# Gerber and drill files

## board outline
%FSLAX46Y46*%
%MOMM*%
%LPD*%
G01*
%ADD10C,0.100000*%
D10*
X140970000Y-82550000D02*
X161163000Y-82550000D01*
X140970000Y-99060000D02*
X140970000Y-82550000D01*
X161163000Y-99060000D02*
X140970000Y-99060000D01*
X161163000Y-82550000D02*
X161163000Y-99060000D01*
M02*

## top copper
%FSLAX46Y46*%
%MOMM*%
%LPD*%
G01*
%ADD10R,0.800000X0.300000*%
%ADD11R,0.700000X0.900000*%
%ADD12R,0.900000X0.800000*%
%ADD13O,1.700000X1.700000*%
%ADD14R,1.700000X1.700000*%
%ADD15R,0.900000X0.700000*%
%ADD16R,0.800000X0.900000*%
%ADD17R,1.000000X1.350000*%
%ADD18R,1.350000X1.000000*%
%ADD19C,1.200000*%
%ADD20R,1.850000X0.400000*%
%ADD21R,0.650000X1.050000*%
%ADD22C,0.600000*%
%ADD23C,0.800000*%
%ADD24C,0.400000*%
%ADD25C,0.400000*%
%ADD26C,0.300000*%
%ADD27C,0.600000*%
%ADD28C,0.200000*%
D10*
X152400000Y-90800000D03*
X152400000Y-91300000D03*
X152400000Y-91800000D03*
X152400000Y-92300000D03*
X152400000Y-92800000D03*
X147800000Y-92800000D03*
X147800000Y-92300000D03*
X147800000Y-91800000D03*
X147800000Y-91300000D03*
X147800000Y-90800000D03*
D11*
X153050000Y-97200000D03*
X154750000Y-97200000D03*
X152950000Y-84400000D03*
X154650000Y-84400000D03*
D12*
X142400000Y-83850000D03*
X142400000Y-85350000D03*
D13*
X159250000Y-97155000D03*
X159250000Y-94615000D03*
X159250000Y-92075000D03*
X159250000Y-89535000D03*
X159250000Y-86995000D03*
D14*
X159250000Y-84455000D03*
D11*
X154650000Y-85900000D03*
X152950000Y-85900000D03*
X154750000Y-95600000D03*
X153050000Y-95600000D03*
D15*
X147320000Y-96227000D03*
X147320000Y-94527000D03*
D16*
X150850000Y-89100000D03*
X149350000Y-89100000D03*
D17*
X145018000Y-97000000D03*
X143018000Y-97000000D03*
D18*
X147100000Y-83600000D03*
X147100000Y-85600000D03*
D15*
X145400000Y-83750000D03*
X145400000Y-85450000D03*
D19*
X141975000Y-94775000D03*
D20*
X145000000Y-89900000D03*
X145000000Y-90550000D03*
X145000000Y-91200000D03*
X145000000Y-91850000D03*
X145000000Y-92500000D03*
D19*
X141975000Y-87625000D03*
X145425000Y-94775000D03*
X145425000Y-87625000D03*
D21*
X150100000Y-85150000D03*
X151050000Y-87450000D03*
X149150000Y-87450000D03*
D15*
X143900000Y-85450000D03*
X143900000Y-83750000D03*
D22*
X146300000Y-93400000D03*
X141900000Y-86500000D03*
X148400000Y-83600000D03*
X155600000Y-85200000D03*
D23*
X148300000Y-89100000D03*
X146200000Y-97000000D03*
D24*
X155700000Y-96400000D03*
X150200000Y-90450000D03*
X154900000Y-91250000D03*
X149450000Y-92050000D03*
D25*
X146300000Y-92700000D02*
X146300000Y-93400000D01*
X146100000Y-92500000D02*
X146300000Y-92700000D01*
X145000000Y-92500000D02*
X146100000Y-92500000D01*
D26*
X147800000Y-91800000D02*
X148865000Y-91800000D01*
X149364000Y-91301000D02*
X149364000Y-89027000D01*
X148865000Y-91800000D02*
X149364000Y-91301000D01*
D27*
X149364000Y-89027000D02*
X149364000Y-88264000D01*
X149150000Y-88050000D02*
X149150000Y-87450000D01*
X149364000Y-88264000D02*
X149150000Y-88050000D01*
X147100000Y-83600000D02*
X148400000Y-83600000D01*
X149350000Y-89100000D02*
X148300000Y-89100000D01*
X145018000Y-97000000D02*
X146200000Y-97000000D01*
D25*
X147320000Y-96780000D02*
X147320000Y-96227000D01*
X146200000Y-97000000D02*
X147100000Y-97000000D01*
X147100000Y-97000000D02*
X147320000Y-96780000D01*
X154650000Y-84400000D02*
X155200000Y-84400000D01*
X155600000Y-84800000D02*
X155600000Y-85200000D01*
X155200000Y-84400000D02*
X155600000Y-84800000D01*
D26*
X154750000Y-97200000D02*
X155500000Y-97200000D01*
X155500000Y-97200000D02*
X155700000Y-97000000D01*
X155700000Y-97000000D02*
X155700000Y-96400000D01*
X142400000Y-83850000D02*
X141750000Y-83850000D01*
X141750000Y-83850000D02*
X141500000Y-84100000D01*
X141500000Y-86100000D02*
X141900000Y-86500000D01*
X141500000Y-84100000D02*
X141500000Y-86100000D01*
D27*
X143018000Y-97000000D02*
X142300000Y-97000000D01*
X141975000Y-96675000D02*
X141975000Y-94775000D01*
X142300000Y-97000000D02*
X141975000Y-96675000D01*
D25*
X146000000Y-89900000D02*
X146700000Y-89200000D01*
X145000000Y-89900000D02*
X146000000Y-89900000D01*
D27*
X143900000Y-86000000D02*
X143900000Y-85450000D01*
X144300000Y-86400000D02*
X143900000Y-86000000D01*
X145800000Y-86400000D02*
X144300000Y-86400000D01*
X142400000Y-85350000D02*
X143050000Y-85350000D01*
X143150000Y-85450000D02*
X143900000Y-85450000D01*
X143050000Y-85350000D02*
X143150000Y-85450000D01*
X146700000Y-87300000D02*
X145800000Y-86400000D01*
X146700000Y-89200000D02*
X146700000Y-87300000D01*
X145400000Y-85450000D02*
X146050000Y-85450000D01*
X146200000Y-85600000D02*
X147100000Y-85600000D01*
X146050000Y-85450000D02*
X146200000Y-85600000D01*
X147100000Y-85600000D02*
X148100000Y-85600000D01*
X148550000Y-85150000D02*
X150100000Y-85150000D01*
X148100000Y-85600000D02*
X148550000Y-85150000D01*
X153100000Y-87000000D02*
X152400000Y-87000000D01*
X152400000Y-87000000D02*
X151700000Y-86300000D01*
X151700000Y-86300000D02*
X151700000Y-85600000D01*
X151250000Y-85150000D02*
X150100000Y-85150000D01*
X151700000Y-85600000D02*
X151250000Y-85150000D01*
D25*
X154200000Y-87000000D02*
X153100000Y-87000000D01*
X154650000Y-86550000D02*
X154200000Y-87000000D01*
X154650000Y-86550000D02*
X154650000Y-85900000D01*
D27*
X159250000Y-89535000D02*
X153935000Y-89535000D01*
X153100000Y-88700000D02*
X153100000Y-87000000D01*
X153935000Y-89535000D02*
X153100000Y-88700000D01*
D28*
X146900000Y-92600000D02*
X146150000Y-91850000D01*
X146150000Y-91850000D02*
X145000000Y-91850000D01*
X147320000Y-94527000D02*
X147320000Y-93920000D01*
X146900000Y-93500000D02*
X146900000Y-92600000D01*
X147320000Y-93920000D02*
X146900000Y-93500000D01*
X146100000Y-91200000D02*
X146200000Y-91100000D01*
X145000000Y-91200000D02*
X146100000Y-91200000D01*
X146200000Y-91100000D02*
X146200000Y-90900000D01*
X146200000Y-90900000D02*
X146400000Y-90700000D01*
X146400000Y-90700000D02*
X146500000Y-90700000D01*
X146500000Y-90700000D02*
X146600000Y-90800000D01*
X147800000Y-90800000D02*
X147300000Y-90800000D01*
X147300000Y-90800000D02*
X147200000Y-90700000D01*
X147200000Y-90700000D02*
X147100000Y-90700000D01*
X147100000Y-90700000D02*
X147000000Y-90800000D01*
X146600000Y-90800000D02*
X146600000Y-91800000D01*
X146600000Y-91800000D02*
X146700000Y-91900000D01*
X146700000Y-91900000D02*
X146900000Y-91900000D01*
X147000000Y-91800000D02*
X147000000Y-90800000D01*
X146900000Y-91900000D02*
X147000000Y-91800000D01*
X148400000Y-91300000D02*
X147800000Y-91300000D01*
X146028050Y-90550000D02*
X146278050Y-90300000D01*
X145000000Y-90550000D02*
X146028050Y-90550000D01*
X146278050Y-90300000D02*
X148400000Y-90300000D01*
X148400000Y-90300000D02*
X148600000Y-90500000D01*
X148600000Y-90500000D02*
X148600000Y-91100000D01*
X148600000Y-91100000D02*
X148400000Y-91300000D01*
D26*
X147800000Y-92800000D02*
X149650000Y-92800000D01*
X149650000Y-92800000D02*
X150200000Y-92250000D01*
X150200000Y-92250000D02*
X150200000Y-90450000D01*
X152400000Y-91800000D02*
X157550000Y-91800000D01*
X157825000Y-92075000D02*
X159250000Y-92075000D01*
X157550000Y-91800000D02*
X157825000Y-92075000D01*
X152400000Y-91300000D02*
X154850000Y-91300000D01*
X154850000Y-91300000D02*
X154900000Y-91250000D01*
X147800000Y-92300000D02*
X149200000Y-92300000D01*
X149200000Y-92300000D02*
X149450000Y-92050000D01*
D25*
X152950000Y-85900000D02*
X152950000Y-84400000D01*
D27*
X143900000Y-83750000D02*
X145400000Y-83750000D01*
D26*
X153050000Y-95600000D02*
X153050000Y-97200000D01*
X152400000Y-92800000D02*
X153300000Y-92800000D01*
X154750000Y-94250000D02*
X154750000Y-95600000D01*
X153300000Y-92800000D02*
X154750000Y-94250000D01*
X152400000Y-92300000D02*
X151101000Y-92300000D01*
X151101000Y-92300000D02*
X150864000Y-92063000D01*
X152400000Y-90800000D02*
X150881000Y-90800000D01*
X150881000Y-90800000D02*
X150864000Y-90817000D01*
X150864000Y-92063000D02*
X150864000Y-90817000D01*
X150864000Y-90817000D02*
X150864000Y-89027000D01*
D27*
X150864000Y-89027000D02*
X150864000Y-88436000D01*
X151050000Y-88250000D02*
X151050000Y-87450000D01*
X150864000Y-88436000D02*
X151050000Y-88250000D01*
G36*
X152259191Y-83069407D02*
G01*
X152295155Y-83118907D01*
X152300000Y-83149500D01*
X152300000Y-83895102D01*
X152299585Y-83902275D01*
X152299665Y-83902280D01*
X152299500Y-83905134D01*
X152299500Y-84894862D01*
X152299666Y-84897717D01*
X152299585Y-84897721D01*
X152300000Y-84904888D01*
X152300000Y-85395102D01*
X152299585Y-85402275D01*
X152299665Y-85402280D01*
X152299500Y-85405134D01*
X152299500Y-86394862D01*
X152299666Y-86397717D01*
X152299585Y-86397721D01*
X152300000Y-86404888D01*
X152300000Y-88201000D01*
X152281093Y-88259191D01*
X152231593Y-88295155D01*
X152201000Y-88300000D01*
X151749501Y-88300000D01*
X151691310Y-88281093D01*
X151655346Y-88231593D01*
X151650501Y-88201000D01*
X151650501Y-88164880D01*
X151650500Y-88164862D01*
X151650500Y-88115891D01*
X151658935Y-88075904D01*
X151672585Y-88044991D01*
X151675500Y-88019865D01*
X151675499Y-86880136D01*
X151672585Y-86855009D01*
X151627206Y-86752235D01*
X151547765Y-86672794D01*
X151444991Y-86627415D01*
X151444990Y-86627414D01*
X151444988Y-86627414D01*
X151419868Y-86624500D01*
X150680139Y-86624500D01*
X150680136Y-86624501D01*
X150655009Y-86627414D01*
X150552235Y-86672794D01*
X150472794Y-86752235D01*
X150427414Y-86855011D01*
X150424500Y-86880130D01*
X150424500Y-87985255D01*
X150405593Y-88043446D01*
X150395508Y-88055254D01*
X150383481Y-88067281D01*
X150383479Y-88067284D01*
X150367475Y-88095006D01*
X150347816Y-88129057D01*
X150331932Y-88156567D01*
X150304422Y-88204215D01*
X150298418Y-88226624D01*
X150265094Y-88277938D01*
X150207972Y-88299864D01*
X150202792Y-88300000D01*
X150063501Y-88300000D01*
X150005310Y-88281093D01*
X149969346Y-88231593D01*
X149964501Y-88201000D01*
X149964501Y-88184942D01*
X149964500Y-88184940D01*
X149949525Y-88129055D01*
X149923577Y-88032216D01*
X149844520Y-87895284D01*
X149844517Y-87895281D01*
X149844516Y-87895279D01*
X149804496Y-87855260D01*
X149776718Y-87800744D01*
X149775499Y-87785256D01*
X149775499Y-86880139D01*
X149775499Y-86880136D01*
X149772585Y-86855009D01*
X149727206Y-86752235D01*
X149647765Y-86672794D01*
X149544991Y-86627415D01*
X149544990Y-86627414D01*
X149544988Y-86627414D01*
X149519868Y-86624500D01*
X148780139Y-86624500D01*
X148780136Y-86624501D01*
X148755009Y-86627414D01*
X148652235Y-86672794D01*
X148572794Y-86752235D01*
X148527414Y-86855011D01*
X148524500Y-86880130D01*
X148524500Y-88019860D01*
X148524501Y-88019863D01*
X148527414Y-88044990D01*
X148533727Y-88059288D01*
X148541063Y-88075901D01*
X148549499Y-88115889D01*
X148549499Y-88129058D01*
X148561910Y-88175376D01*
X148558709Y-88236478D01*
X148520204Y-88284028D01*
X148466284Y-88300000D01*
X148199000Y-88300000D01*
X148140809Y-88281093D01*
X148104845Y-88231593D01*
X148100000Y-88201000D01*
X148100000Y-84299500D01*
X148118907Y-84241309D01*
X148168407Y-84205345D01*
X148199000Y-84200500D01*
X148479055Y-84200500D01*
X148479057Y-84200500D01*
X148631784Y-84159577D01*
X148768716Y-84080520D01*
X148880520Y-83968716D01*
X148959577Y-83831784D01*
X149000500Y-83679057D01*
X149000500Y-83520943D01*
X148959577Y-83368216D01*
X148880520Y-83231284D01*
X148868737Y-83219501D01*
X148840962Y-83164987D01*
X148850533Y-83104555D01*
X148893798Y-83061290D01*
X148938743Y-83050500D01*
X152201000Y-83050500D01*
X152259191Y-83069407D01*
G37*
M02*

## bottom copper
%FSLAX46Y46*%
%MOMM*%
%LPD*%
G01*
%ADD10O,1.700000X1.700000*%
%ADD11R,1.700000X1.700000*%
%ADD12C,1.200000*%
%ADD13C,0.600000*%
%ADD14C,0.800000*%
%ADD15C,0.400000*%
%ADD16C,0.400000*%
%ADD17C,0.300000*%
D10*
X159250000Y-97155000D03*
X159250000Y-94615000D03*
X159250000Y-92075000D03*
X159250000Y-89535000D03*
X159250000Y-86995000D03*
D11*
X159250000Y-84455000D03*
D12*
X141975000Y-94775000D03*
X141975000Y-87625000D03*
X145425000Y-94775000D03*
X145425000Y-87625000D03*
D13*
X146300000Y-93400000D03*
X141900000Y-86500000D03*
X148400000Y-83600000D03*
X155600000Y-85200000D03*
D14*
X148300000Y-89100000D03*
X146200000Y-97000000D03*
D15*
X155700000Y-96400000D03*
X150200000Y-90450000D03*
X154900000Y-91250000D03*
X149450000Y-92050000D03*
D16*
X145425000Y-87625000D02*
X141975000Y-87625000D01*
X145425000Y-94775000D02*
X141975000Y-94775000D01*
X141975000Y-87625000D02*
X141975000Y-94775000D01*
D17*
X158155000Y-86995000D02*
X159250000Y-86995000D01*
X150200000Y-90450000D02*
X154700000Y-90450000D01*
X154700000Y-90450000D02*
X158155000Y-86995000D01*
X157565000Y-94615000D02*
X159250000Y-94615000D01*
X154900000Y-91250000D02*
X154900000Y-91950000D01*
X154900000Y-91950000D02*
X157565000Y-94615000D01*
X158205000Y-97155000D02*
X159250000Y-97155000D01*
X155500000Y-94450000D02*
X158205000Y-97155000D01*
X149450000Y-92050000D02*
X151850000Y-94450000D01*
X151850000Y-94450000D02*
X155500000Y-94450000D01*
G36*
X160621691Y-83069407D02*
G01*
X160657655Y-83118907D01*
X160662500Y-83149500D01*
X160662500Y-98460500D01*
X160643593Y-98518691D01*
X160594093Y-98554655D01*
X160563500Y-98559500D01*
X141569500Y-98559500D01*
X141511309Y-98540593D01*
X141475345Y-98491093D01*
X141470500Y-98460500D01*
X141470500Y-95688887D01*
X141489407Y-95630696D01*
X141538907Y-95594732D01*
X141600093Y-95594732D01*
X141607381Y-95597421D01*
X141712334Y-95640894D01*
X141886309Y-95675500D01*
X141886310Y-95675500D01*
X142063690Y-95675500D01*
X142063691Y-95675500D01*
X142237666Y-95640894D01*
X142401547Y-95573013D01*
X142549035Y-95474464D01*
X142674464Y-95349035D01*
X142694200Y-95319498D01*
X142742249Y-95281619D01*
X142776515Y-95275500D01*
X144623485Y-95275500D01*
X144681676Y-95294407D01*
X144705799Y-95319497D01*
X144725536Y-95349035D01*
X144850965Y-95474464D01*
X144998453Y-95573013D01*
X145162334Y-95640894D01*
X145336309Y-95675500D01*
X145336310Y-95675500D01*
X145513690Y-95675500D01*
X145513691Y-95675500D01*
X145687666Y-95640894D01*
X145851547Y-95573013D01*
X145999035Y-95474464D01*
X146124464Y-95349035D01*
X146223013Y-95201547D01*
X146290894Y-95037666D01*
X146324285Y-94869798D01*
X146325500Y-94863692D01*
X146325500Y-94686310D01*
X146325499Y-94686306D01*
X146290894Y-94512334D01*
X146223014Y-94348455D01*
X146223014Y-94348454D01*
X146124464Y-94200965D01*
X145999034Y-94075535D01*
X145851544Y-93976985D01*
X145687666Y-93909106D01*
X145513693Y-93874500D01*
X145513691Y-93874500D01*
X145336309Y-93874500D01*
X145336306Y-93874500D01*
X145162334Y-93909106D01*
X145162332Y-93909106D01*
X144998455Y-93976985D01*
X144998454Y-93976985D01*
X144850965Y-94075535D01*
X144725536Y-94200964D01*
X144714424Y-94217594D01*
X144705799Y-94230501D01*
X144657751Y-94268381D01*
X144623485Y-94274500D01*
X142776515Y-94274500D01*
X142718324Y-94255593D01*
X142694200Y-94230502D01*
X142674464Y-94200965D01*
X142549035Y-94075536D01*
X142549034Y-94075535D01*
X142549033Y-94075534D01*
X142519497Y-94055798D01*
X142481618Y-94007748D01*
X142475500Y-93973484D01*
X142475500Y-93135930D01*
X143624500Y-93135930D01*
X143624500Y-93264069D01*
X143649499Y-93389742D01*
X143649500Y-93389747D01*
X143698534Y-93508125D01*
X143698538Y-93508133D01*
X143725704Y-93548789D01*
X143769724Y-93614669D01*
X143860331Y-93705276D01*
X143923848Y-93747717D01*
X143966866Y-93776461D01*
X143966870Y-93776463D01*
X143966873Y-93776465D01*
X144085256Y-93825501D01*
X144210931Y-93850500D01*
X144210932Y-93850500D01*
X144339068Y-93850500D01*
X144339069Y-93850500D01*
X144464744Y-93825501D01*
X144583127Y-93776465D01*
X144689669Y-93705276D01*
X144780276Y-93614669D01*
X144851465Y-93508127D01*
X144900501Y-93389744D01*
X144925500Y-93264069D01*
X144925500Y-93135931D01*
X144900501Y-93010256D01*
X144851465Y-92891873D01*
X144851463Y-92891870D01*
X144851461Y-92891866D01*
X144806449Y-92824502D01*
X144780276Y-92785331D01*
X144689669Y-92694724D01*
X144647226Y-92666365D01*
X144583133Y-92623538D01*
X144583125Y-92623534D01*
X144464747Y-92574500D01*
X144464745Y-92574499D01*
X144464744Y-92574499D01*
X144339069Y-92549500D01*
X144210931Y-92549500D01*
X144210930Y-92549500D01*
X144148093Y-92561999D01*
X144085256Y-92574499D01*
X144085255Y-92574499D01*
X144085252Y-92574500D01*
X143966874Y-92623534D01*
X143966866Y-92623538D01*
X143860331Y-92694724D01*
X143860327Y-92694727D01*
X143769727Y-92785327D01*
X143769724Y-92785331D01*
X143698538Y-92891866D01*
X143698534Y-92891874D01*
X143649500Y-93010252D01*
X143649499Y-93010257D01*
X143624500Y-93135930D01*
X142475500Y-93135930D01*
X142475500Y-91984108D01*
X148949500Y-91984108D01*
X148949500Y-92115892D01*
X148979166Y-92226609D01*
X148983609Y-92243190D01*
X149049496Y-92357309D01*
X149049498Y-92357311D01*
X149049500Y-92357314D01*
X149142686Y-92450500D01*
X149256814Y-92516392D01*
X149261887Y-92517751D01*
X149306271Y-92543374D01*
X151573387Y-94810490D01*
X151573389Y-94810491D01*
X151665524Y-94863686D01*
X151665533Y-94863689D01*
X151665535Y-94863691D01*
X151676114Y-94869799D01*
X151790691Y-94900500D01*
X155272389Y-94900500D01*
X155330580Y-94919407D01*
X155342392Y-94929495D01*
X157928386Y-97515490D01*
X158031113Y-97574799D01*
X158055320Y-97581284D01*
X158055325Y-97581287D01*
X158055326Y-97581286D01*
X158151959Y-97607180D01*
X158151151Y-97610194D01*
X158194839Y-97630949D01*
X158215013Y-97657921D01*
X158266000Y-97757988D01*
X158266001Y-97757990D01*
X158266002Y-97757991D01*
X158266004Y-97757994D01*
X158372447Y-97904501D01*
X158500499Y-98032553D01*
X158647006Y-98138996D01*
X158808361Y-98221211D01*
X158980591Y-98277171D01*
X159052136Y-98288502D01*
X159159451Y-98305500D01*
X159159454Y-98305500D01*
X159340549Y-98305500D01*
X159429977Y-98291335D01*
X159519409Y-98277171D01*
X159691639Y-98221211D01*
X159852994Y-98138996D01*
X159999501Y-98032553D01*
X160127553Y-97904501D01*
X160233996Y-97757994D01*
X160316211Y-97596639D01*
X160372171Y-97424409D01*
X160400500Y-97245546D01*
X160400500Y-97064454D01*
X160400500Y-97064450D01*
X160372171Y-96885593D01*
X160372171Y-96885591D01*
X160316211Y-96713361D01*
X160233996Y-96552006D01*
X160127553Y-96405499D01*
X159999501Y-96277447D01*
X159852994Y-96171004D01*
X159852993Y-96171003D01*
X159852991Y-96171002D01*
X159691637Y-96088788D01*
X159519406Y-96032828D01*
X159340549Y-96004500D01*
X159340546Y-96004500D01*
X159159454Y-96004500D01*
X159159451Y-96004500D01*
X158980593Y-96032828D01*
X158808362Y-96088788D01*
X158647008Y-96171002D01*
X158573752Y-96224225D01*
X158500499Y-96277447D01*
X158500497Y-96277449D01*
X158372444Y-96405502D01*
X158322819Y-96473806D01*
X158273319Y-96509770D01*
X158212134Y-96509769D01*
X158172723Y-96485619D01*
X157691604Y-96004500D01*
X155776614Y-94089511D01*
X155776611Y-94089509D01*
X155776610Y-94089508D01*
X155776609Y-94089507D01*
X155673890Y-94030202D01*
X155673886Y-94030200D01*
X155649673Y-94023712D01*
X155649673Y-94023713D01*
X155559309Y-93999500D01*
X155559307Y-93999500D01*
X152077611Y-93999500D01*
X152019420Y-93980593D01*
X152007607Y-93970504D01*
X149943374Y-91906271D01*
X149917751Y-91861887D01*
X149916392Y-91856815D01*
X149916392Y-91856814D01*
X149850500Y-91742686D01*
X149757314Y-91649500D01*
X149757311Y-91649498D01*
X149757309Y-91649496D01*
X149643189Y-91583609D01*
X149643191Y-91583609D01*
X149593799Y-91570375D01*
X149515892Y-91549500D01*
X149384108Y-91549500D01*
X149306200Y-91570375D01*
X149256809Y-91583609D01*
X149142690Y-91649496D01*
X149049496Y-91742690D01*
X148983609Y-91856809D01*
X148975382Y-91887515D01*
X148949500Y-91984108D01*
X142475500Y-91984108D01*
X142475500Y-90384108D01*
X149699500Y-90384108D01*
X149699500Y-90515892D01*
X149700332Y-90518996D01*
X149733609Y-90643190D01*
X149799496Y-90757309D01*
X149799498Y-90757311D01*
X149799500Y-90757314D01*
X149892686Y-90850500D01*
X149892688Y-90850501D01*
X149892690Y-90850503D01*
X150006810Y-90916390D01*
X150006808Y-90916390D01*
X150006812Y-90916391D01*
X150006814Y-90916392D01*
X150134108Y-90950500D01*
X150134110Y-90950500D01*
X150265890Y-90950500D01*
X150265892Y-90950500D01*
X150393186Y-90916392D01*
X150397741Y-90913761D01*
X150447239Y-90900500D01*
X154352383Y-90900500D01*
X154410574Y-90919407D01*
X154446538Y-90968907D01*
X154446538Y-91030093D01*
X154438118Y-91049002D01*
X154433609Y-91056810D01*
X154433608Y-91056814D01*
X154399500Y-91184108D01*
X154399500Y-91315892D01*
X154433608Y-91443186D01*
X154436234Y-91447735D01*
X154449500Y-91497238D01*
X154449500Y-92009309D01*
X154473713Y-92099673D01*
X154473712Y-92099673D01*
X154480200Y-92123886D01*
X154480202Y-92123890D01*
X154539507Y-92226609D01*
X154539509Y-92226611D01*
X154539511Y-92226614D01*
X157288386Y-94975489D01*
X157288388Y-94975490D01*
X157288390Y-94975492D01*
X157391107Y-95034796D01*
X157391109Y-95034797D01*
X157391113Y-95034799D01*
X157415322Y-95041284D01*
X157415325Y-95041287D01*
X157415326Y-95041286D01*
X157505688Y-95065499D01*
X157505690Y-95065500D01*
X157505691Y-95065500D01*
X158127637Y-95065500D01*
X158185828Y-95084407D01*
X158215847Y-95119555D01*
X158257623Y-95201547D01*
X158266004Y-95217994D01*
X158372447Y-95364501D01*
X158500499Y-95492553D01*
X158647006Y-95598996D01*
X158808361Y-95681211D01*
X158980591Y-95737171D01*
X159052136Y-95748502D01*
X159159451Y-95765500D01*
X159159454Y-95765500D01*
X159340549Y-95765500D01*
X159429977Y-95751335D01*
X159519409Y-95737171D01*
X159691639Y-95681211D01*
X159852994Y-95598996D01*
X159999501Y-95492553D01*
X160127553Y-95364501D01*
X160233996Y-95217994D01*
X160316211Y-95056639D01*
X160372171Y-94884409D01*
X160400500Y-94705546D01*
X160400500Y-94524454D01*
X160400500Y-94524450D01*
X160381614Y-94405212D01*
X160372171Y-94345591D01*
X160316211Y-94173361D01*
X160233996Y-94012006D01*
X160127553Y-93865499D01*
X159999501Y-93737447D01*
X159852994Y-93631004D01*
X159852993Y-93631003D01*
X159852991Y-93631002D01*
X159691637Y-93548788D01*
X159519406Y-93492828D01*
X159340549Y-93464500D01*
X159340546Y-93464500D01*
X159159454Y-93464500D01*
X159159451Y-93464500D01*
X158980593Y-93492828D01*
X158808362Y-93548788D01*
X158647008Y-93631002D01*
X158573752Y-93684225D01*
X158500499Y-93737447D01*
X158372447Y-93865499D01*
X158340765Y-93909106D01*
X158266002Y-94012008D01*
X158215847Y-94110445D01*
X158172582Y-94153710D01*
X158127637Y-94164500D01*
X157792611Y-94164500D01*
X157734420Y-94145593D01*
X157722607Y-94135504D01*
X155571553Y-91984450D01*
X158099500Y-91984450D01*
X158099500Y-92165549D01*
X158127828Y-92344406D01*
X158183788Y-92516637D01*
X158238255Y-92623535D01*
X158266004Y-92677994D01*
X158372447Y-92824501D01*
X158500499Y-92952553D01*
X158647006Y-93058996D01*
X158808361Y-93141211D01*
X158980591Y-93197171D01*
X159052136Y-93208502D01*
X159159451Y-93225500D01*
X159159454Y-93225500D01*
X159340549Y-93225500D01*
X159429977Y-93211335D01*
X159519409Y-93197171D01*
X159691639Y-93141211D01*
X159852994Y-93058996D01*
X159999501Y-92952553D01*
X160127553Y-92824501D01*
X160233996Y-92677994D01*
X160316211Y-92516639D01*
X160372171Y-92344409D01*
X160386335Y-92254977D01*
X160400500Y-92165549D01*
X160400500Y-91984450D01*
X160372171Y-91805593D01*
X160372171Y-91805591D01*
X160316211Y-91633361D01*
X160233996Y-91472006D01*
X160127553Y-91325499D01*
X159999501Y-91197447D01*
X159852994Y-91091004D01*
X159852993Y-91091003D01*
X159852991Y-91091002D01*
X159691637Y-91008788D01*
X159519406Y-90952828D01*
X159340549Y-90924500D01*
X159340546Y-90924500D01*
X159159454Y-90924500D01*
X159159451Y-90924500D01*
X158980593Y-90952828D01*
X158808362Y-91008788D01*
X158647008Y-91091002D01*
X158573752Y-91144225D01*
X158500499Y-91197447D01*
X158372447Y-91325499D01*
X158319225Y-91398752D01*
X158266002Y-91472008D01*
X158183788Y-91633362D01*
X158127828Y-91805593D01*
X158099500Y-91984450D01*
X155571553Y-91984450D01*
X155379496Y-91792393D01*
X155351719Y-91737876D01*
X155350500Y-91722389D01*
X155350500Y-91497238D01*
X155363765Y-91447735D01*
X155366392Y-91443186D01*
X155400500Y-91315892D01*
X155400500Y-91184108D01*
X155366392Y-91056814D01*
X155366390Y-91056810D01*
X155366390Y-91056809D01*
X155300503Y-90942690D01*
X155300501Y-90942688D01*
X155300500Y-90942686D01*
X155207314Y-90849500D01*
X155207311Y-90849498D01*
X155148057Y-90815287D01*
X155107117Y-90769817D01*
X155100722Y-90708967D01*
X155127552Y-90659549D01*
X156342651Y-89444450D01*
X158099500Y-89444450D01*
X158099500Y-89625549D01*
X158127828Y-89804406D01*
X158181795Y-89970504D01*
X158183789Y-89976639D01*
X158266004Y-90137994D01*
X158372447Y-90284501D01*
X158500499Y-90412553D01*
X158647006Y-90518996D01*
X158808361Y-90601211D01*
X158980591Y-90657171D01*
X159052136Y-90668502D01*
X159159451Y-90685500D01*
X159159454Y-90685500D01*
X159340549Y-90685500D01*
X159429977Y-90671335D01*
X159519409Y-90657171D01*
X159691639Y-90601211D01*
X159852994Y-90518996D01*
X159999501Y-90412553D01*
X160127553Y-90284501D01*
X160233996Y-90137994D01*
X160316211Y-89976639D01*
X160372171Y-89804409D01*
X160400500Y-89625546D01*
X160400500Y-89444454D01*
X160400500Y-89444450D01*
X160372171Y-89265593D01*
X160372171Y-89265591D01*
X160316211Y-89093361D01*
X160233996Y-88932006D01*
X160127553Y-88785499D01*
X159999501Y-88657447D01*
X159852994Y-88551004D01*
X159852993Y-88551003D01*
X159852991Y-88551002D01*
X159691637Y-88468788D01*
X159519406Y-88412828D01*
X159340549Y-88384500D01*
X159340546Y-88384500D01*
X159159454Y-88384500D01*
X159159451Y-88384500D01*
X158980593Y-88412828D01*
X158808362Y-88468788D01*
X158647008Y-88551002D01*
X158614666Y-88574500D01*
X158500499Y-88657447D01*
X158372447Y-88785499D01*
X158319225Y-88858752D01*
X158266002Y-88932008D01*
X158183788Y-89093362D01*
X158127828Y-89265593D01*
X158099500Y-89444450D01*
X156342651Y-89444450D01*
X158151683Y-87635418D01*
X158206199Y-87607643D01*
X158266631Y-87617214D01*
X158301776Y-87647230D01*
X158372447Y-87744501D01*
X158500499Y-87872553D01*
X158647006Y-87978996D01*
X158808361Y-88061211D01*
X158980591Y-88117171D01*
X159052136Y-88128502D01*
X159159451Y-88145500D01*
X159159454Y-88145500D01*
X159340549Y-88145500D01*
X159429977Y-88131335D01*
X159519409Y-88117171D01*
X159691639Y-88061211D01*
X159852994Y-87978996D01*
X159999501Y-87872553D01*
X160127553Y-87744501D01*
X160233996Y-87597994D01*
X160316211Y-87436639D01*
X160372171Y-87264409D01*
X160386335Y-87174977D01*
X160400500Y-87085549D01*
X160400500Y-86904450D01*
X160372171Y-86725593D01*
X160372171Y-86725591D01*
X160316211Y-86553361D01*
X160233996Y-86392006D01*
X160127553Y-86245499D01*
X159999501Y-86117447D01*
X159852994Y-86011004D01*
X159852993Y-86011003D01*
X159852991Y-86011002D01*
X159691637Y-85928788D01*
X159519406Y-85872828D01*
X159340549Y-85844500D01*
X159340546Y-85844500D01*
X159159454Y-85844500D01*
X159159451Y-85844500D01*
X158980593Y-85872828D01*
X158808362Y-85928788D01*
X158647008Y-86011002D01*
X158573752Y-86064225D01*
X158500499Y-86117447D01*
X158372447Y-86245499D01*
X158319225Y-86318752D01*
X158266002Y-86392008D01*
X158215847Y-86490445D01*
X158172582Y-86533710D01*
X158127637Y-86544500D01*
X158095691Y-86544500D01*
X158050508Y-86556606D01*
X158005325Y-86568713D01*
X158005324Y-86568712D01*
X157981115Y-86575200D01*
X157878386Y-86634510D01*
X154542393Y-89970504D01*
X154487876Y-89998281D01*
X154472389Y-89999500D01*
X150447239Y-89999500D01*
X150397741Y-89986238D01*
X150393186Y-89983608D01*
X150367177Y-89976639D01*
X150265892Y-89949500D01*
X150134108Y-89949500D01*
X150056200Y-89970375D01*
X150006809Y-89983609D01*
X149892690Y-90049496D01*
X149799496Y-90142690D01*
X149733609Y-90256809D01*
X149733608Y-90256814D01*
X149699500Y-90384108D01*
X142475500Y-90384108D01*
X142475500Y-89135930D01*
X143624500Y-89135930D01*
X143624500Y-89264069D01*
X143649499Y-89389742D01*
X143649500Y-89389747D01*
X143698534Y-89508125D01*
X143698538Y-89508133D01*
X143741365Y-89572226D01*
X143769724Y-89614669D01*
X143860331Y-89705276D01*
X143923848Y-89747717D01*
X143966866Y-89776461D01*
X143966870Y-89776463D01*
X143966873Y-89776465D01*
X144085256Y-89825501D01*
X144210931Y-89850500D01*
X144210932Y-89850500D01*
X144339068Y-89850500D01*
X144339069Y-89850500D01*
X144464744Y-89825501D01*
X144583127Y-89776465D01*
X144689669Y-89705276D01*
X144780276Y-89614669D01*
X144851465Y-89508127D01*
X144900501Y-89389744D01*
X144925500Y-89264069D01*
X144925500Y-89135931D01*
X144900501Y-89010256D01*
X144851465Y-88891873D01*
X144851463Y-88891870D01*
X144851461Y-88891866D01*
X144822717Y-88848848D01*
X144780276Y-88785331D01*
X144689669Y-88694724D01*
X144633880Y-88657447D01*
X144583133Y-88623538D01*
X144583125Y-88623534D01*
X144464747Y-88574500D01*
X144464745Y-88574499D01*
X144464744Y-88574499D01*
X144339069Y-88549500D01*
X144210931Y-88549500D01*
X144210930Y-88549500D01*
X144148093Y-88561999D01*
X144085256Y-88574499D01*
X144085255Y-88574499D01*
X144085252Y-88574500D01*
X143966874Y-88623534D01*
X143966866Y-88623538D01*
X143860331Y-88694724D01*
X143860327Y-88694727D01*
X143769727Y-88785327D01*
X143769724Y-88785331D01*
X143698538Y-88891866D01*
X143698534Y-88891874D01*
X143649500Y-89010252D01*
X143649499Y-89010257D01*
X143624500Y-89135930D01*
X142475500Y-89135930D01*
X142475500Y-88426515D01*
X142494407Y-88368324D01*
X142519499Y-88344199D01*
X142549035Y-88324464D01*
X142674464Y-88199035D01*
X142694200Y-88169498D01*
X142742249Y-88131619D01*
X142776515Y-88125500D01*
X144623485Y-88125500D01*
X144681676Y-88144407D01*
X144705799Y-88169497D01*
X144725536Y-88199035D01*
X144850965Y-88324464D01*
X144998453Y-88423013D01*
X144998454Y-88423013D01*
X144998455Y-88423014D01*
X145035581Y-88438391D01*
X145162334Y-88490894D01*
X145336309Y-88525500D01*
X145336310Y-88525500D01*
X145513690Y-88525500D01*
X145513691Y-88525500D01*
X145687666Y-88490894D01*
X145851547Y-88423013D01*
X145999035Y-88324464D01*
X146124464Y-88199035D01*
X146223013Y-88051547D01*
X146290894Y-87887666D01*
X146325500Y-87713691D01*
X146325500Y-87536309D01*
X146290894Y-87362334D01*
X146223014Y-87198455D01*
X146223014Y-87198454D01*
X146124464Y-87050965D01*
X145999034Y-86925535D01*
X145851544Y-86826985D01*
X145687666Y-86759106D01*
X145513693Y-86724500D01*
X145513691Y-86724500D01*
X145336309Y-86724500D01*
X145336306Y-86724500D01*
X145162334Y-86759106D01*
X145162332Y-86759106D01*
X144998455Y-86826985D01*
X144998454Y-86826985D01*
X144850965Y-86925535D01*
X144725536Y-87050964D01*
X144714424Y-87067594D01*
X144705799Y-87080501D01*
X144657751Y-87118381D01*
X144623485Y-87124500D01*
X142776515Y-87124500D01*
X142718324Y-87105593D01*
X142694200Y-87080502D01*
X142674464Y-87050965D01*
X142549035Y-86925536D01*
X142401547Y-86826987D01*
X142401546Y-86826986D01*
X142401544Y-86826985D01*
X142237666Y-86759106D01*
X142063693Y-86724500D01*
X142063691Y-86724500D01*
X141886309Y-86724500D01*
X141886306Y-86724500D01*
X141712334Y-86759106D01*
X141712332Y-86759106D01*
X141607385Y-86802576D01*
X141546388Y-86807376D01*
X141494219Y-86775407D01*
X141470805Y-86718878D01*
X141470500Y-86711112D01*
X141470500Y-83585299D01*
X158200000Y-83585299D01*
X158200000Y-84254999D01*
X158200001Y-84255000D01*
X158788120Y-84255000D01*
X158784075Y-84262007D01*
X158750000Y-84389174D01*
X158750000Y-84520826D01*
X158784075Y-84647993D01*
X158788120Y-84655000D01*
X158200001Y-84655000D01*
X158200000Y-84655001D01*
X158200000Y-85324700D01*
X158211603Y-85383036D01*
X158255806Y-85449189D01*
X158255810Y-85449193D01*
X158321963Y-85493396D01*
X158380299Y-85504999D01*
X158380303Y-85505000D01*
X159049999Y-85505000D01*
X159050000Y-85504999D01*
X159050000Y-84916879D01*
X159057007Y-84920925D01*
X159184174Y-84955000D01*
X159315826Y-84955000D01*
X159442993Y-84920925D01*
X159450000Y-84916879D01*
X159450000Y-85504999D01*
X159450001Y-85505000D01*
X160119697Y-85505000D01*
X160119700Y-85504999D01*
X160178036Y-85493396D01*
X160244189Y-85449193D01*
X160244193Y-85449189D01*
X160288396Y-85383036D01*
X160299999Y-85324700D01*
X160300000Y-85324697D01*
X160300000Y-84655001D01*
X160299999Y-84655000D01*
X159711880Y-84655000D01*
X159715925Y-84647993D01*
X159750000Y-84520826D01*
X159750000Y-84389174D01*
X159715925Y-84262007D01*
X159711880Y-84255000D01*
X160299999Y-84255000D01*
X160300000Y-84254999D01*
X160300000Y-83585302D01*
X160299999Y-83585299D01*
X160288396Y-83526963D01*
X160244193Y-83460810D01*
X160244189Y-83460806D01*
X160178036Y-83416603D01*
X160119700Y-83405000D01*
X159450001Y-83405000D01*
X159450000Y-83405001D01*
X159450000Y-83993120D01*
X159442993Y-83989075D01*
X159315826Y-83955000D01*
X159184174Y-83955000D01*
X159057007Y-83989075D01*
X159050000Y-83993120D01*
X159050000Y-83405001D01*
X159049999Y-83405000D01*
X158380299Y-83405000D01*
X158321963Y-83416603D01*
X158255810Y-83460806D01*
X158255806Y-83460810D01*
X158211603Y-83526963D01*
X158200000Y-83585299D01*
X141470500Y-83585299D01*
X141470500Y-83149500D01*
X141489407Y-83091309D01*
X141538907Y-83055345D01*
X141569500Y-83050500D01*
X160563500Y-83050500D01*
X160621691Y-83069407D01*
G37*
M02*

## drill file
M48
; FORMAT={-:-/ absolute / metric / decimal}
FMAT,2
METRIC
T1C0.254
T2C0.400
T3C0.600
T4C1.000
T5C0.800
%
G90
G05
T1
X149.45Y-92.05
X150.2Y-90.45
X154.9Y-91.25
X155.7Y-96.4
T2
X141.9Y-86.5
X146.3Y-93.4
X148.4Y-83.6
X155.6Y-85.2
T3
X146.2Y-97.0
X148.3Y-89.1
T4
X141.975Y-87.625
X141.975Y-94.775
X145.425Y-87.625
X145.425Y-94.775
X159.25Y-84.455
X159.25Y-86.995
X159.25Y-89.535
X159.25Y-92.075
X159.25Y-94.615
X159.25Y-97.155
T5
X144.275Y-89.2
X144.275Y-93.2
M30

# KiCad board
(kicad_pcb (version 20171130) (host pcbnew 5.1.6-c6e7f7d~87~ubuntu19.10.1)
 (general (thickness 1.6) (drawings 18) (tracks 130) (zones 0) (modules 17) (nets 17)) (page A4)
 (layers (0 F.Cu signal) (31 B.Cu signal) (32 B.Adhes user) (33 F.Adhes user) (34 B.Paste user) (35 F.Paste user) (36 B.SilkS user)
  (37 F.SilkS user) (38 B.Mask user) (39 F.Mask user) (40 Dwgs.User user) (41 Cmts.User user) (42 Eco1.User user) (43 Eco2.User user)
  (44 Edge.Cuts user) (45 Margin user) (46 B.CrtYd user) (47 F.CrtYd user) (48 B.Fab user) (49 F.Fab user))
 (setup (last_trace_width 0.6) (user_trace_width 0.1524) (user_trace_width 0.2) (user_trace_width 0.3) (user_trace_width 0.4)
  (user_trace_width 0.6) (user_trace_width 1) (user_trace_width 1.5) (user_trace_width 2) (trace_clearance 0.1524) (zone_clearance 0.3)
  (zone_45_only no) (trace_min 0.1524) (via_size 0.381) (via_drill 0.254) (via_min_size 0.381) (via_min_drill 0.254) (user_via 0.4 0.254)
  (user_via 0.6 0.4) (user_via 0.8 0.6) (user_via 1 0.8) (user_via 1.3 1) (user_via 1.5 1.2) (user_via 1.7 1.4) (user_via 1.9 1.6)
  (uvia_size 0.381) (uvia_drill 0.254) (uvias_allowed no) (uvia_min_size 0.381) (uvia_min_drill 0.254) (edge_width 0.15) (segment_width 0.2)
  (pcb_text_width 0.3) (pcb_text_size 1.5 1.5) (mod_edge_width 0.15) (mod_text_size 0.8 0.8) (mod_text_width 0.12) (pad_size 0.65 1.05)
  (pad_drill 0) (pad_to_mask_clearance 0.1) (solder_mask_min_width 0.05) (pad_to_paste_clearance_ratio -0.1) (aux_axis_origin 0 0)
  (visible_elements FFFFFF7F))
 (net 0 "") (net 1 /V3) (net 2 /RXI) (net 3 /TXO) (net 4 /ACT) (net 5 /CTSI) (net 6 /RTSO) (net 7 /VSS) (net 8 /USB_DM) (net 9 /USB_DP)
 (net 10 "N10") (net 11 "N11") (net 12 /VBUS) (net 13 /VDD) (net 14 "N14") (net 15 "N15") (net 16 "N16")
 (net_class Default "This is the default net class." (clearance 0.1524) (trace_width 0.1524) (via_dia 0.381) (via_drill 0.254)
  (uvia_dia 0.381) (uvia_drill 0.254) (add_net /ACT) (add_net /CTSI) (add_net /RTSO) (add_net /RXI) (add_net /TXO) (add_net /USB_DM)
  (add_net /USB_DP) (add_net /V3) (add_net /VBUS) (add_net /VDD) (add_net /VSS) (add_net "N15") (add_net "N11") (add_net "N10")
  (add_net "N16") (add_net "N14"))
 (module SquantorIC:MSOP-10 (layer F.Cu) (at 150.1 91.8)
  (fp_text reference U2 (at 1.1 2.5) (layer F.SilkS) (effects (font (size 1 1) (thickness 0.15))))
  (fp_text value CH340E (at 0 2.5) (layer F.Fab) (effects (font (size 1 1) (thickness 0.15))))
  (pad 10 smd rect (at 2.3 -1) (size 0.8 0.3) (layers F.Cu F.Paste F.Mask) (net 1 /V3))
  (pad 9 smd rect (at 2.3 -0.5) (size 0.8 0.3) (layers F.Cu F.Paste F.Mask) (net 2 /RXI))
  (pad 8 smd rect (at 2.3 0) (size 0.8 0.3) (layers F.Cu F.Paste F.Mask) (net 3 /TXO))
  (pad 7 smd rect (at 2.3 0.5) (size 0.8 0.3) (layers F.Cu F.Paste F.Mask) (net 1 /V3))
  (pad 6 smd rect (at 2.3 1) (size 0.8 0.3) (layers F.Cu F.Paste F.Mask) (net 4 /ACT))
  (pad 5 smd rect (at -2.3 1) (size 0.8 0.3) (layers F.Cu F.Paste F.Mask) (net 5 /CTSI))
  (pad 4 smd rect (at -2.3 0.5) (size 0.8 0.3) (layers F.Cu F.Paste F.Mask) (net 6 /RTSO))
  (pad 3 smd rect (at -2.3 0) (size 0.8 0.3) (layers F.Cu F.Paste F.Mask) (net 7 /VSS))
  (pad 2 smd rect (at -2.3 -0.5) (size 0.8 0.3) (layers F.Cu F.Paste F.Mask) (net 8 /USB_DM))
  (pad 1 smd rect (at -2.3 -1) (size 0.8 0.3) (layers F.Cu F.Paste F.Mask) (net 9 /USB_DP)))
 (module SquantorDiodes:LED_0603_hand (layer F.Cu) (at 153.9 97.2 180)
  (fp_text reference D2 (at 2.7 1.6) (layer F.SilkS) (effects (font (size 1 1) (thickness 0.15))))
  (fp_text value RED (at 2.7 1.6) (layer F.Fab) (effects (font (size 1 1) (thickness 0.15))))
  (pad 2 smd rect (at 0.85 0 180) (size 0.7 0.9) (layers F.Cu F.Paste F.Mask) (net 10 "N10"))
  (pad 1 smd rect (at -0.85 0 180) (size 0.7 0.9) (layers F.Cu F.Paste F.Mask) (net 7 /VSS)))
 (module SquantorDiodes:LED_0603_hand (layer F.Cu) (at 153.8 84.4 180)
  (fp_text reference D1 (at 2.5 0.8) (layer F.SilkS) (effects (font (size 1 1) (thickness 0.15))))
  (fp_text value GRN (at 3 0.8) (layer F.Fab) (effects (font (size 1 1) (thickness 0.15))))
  (pad 2 smd rect (at 0.85 0 180) (size 0.7 0.9) (layers F.Cu F.Paste F.Mask) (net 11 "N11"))
  (pad 1 smd rect (at -0.85 0 180) (size 0.7 0.9) (layers F.Cu F.Paste F.Mask) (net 7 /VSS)))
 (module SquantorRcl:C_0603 (layer F.Cu) (at 142.4 84.6 90)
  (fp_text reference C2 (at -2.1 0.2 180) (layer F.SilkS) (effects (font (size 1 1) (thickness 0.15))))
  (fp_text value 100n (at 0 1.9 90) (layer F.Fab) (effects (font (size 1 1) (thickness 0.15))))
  (pad 2 smd rect (at 0.75 0 90) (size 0.8 0.9) (layers F.Cu F.Paste F.Mask) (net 7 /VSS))
  (pad 1 smd rect (at -0.75 0 90) (size 0.8 0.9) (layers F.Cu F.Paste F.Mask) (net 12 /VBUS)))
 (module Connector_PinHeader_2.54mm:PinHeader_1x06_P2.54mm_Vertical (layer F.Cu) (at 159.25 84.455)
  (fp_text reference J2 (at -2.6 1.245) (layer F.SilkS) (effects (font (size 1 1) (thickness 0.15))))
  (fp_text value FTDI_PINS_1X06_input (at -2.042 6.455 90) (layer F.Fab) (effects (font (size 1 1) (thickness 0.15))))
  (pad 6 thru_hole oval (at 0 12.7) (size 1.7 1.7) (drill 1) (layers *.Cu *.Mask) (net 6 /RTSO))
  (pad 5 thru_hole oval (at 0 10.16) (size 1.7 1.7) (drill 1) (layers *.Cu *.Mask) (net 2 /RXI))
  (pad 4 thru_hole oval (at 0 7.62) (size 1.7 1.7) (drill 1) (layers *.Cu *.Mask) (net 3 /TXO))
  (pad 3 thru_hole oval (at 0 5.08) (size 1.7 1.7) (drill 1) (layers *.Cu *.Mask) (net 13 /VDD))
  (pad 2 thru_hole oval (at 0 2.54) (size 1.7 1.7) (drill 1) (layers *.Cu *.Mask) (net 5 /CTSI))
  (pad 1 thru_hole rect (at 0 0) (size 1.7 1.7) (drill 1) (layers *.Cu *.Mask) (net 7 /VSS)))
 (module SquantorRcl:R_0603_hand (layer F.Cu) (at 153.8 85.9)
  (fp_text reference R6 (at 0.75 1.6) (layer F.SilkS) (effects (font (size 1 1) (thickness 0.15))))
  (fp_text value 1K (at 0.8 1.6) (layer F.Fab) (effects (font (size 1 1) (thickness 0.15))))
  (pad 2 smd rect (at 0.85 0) (size 0.7 0.9) (layers F.Cu F.Paste F.Mask) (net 13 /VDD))
  (pad 1 smd rect (at -0.85 0) (size 0.7 0.9) (layers F.Cu F.Paste F.Mask) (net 11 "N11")))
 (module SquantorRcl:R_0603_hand (layer F.Cu) (at 153.9 95.6)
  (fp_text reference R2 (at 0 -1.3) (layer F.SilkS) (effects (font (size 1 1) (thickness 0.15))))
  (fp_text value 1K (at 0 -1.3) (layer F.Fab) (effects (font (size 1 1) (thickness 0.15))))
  (pad 2 smd rect (at 0.85 0) (size 0.7 0.9) (layers F.Cu F.Paste F.Mask) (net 4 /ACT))
  (pad 1 smd rect (at -0.85 0) (size 0.7 0.9) (layers F.Cu F.Paste F.Mask) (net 10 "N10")))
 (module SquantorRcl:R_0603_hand (layer F.Cu) (at 147.32 95.377 270)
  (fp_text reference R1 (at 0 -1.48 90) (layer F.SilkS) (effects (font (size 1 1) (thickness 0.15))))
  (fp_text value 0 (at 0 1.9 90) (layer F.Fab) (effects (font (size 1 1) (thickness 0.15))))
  (pad 2 smd rect (at 0.85 0 270) (size 0.7 0.9) (layers F.Cu F.Paste F.Mask) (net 7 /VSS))
  (pad 1 smd rect (at -0.85 0 270) (size 0.7 0.9) (layers F.Cu F.Paste F.Mask) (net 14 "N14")))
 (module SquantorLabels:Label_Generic (layer B.Cu) (at 151.4 95.6 180)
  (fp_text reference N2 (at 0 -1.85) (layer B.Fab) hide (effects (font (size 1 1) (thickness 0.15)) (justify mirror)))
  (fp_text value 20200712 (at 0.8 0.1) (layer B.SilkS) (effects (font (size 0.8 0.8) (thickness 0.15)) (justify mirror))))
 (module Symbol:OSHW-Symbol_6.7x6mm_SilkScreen (layer B.Cu) (at 150.6 91.8 180)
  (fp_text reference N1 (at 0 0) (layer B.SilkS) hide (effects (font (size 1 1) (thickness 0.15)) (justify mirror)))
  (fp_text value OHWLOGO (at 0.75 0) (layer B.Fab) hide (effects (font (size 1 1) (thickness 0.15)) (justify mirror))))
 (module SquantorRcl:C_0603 (layer F.Cu) (at 150.1 89.1)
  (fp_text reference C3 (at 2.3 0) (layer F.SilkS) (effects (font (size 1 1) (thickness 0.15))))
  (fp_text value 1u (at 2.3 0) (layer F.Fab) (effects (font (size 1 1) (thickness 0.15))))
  (pad 2 smd rect (at 0.75 0) (size 0.8 0.9) (layers F.Cu F.Paste F.Mask) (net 1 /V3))
  (pad 1 smd rect (at -0.75 0) (size 0.8 0.9) (layers F.Cu F.Paste F.Mask) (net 7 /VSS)))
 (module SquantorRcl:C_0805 (layer F.Cu) (at 144.018 97)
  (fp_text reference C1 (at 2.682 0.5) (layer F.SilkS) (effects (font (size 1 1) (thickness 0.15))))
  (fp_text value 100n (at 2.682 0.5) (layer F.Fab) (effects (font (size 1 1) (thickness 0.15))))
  (pad 2 smd rect (at 1 0) (size 1 1.35) (layers F.Cu F.Paste F.Mask) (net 7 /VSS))
  (pad 1 smd rect (at -1 0) (size 1 1.35) (layers F.Cu F.Paste F.Mask) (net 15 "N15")))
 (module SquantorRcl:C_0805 (layer F.Cu) (at 147.1 84.6 90)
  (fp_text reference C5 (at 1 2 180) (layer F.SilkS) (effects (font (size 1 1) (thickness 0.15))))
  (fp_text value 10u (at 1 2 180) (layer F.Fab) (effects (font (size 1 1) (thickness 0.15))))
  (pad 2 smd rect (at 1 0 90) (size 1 1.35) (layers F.Cu F.Paste F.Mask) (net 7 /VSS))
  (pad 1 smd rect (at -1 0 90) (size 1 1.35) (layers F.Cu F.Paste F.Mask) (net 13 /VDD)))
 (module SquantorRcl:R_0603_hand (layer F.Cu) (at 145.4 84.6 90)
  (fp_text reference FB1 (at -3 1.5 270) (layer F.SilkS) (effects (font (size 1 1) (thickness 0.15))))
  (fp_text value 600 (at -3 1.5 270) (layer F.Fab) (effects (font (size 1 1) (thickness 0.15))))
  (pad 2 smd rect (at 0.85 0 90) (size 0.7 0.9) (layers F.Cu F.Paste F.Mask) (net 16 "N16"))
  (pad 1 smd rect (at -0.85 0 90) (size 0.7 0.9) (layers F.Cu F.Paste F.Mask) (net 13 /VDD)))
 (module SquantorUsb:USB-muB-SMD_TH (layer F.Cu) (at 143.7 91.2 270)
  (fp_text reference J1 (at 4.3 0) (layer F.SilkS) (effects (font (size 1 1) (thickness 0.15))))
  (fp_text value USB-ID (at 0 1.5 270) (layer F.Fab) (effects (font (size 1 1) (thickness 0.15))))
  (pad S thru_hole circle (at 3.575 1.725 270) (size 1.2 1.2) (drill 1) (layers *.Cu *.Mask) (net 15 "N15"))
  (pad "" np_thru_hole circle (at 2 -0.575 270) (size 0.8 0.8) (drill 0.8) (layers *.Cu))
  (pad 1 smd rect (at -1.3 -1.3 270) (size 0.4 1.85) (layers F.Cu F.Paste F.Mask) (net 12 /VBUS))
  (pad 2 smd rect (at -0.65 -1.3 270) (size 0.4 1.85) (layers F.Cu F.Paste F.Mask) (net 8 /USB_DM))
  (pad 3 smd rect (at 0 -1.3 270) (size 0.4 1.85) (layers F.Cu F.Paste F.Mask) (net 9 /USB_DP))
  (pad 4 smd rect (at 0.65 -1.3 270) (size 0.4 1.85) (layers F.Cu F.Paste F.Mask) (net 14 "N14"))
  (pad 5 smd rect (at 1.3 -1.3 270) (size 0.4 1.85) (layers F.Cu F.Paste F.Mask) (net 7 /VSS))
  (pad "" np_thru_hole circle (at -2 -0.575 270) (size 0.8 0.8) (drill 0.8) (layers *.Cu))
  (pad S thru_hole circle (at -3.575 1.725 270) (size 1.2 1.2) (drill 1) (layers *.Cu *.Mask) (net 15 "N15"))
  (pad S thru_hole circle (at 3.575 -1.725 270) (size 1.2 1.2) (drill 1) (layers *.Cu *.Mask) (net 15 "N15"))
  (pad S thru_hole circle (at -3.575 -1.725 270) (size 1.2 1.2) (drill 1) (layers *.Cu *.Mask) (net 15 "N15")))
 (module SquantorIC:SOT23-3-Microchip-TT (layer F.Cu) (at 150.1 86.3)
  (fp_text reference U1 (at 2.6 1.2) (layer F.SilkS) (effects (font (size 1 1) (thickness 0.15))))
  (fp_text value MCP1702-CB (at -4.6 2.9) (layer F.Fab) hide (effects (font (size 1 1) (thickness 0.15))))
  (pad 3 smd rect (at 0 -1.15) (size 0.65 1.05) (layers F.Cu F.Paste F.Mask) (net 13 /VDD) (zone_connect 2))
  (pad 2 smd rect (at 0.95 1.15) (size 0.65 1.05) (layers F.Cu F.Paste F.Mask) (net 1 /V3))
  (pad 1 smd rect (at -0.95 1.15) (size 0.65 1.05) (layers F.Cu F.Paste F.Mask) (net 7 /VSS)))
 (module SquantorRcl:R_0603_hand (layer F.Cu) (at 143.9 84.6 270)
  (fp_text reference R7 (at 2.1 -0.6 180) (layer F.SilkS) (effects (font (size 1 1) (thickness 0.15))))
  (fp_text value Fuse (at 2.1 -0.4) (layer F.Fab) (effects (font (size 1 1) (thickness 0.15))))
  (pad 2 smd rect (at 0.85 0 270) (size 0.7 0.9) (layers F.Cu F.Paste F.Mask) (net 12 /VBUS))
  (pad 1 smd rect (at -0.85 0 270) (size 0.7 0.9) (layers F.Cu F.Paste F.Mask) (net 16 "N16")))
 (gr_line (start 140.97 82.55) (end 161.163 82.55) (layer Edge.Cuts) (width 0.1))
 (gr_line (start 140.97 99.06) (end 140.97 82.55) (layer Edge.Cuts) (width 0.1))
 (gr_line (start 161.163 99.06) (end 140.97 99.06) (layer Edge.Cuts) (width 0.1))
 (gr_line (start 161.163 82.55) (end 161.163 99.06) (layer Edge.Cuts) (width 0.1))
 (segment (start 146.3 92.7) (end 146.3 93.4) (width 0.4) (layer F.Cu) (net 7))
 (segment (start 146.1 92.5) (end 146.3 92.7) (width 0.4) (layer F.Cu) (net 7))
 (segment (start 145 92.5) (end 146.1 92.5) (width 0.4) (layer F.Cu) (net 7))
 (via (at 146.3 93.4) (size 0.6) (drill 0.4) (layers F.Cu B.Cu) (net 7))
 (segment (start 147.8 91.8) (end 148.865 91.8) (width 0.3) (layer F.Cu) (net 7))
 (segment (start 149.364 91.301) (end 149.364 89.027) (width 0.3) (layer F.Cu) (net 7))
 (segment (start 148.865 91.8) (end 149.364 91.301) (width 0.3) (layer F.Cu) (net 7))
 (segment (start 149.364 89.027) (end 149.364 88.264) (width 0.6) (layer F.Cu) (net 7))
 (segment (start 149.15 88.05) (end 149.15 87.45) (width 0.6) (layer F.Cu) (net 7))
 (segment (start 149.364 88.264) (end 149.15 88.05) (width 0.6) (layer F.Cu) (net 7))
 (via (at 141.9 86.5) (size 0.6) (drill 0.4) (layers F.Cu B.Cu) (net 7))
 (via (at 148.4 83.6) (size 0.6) (drill 0.4) (layers F.Cu B.Cu) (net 7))
 (segment (start 147.1 83.6) (end 148.4 83.6) (width 0.6) (layer F.Cu) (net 7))
 (via (at 155.6 85.2) (size 0.6) (drill 0.4) (layers F.Cu B.Cu) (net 7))
 (via (at 148.3 89.1) (size 0.8) (drill 0.6) (layers F.Cu B.Cu) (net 7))
 (segment (start 149.35 89.1) (end 148.3 89.1) (width 0.6) (layer F.Cu) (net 7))
 (via (at 146.2 97) (size 0.8) (drill 0.6) (layers F.Cu B.Cu) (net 7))
 (segment (start 145.018 97) (end 146.2 97) (width 0.6) (layer F.Cu) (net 7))
 (segment (start 147.32 96.78) (end 147.32 96.227) (width 0.4) (layer F.Cu) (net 7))
 (segment (start 146.2 97) (end 147.1 97) (width 0.4) (layer F.Cu) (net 7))
 (segment (start 147.1 97) (end 147.32 96.78) (width 0.4) (layer F.Cu) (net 7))
 (segment (start 154.65 84.4) (end 155.2 84.4) (width 0.4) (layer F.Cu) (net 7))
 (segment (start 155.6 84.8) (end 155.6 85.2) (width 0.4) (layer F.Cu) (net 7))
 (segment (start 155.2 84.4) (end 155.6 84.8) (width 0.4) (layer F.Cu) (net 7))
 (segment (start 154.75 97.2) (end 155.5 97.2) (width 0.3) (layer F.Cu) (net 7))
 (via (at 155.7 96.4) (size 0.4) (drill 0.254) (layers F.Cu B.Cu) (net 7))
 (segment (start 155.5 97.2) (end 155.7 97) (width 0.3) (layer F.Cu) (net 7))
 (segment (start 155.7 97) (end 155.7 96.4) (width 0.3) (layer F.Cu) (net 7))
 (segment (start 142.4 83.85) (end 141.75 83.85) (width 0.3) (layer F.Cu) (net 7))
 (segment (start 141.75 83.85) (end 141.5 84.1) (width 0.3) (layer F.Cu) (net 7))
 (segment (start 141.5 86.1) (end 141.9 86.5) (width 0.3) (layer F.Cu) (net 7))
 (segment (start 141.5 84.1) (end 141.5 86.1) (width 0.3) (layer F.Cu) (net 7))
 (segment (start 145.425 87.625) (end 141.975 87.625) (width 0.4) (layer B.Cu) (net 15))
 (segment (start 145.425 94.775) (end 141.975 94.775) (width 0.4) (layer B.Cu) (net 15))
 (segment (start 141.975 87.625) (end 141.975 94.775) (width 0.4) (layer B.Cu) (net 15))
 (segment (start 143.018 97) (end 142.3 97) (width 0.6) (layer F.Cu) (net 15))
 (segment (start 141.975 96.675) (end 141.975 94.775) (width 0.6) (layer F.Cu) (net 15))
 (segment (start 142.3 97) (end 141.975 96.675) (width 0.6) (layer F.Cu) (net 15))
 (segment (start 146 89.9) (end 146.7 89.2) (width 0.4) (layer F.Cu) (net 12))
 (segment (start 145 89.9) (end 146 89.9) (width 0.4) (layer F.Cu) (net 12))
 (segment (start 143.9 86) (end 143.9 85.45) (width 0.6) (layer F.Cu) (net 12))
 (segment (start 144.3 86.4) (end 143.9 86) (width 0.6) (layer F.Cu) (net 12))
 (segment (start 145.8 86.4) (end 144.3 86.4) (width 0.6) (layer F.Cu) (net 12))
 (segment (start 142.4 85.35) (end 143.05 85.35) (width 0.6) (layer F.Cu) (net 12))
 (segment (start 143.15 85.45) (end 143.9 85.45) (width 0.6) (layer F.Cu) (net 12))
 (segment (start 143.05 85.35) (end 143.15 85.45) (width 0.6) (layer F.Cu) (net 12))
 (segment (start 146.7 87.3) (end 145.8 86.4) (width 0.6) (layer F.Cu) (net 12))
 (segment (start 146.7 89.2) (end 146.7 87.3) (width 0.6) (layer F.Cu) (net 12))
 (segment (start 145.4 85.45) (end 146.05 85.45) (width 0.6) (layer F.Cu) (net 13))
 (segment (start 146.2 85.6) (end 147.1 85.6) (width 0.6) (layer F.Cu) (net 13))
 (segment (start 146.05 85.45) (end 146.2 85.6) (width 0.6) (layer F.Cu) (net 13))
 (segment (start 147.1 85.6) (end 148.1 85.6) (width 0.6) (layer F.Cu) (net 13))
 (segment (start 148.55 85.15) (end 150.1 85.15) (width 0.6) (layer F.Cu) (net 13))
 (segment (start 148.1 85.6) (end 148.55 85.15) (width 0.6) (layer F.Cu) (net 13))
 (segment (start 153.1 87) (end 152.4 87) (width 0.6) (layer F.Cu) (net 13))
 (segment (start 152.4 87) (end 151.7 86.3) (width 0.6) (layer F.Cu) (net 13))
 (segment (start 151.7 86.3) (end 151.7 85.6) (width 0.6) (layer F.Cu) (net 13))
 (segment (start 151.25 85.15) (end 150.1 85.15) (width 0.6) (layer F.Cu) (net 13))
 (segment (start 151.7 85.6) (end 151.25 85.15) (width 0.6) (layer F.Cu) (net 13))
 (segment (start 154.2 87) (end 153.1 87) (width 0.4) (layer F.Cu) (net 13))
 (segment (start 154.65 86.55) (end 154.2 87) (width 0.4) (layer F.Cu) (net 13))
 (segment (start 154.65 86.55) (end 154.65 85.9) (width 0.4) (layer F.Cu) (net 13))
 (segment (start 159.25 89.535) (end 153.935 89.535) (width 0.6) (layer F.Cu) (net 13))
 (segment (start 153.1 88.7) (end 153.1 87) (width 0.6) (layer F.Cu) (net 13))
 (segment (start 153.935 89.535) (end 153.1 88.7) (width 0.6) (layer F.Cu) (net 13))
 (segment (start 146.9 92.6) (end 146.15 91.85) (width 0.2) (layer F.Cu) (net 14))
 (segment (start 146.15 91.85) (end 145 91.85) (width 0.2) (layer F.Cu) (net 14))
 (segment (start 147.32 94.527) (end 147.32 93.92) (width 0.2) (layer F.Cu) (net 14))
 (segment (start 146.9 93.5) (end 146.9 92.6) (width 0.2) (layer F.Cu) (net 14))
 (segment (start 147.32 93.92) (end 146.9 93.5) (width 0.2) (layer F.Cu) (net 14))
 (segment (start 146.1 91.2) (end 146.2 91.1) (width 0.2) (layer F.Cu) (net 9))
 (segment (start 145 91.2) (end 146.1 91.2) (width 0.2) (layer F.Cu) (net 9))
 (segment (start 146.2 91.1) (end 146.2 90.9) (width 0.2) (layer F.Cu) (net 9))
 (segment (start 146.2 90.9) (end 146.4 90.7) (width 0.2) (layer F.Cu) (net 9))
 (segment (start 146.4 90.7) (end 146.5 90.7) (width 0.2) (layer F.Cu) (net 9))
 (segment (start 146.5 90.7) (end 146.6 90.8) (width 0.2) (layer F.Cu) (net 9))
 (segment (start 147.8 90.8) (end 147.3 90.8) (width 0.2) (layer F.Cu) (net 9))
 (segment (start 147.3 90.8) (end 147.2 90.7) (width 0.2) (layer F.Cu) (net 9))
 (segment (start 147.2 90.7) (end 147.1 90.7) (width 0.2) (layer F.Cu) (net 9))
 (segment (start 147.1 90.7) (end 147 90.8) (width 0.2) (layer F.Cu) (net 9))
 (segment (start 146.6 90.8) (end 146.6 91.8) (width 0.2) (layer F.Cu) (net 9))
 (segment (start 146.6 91.8) (end 146.7 91.9) (width 0.2) (layer F.Cu) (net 9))
 (segment (start 146.7 91.9) (end 146.9 91.9) (width 0.2) (layer F.Cu) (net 9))
 (segment (start 147 91.8) (end 147 90.8) (width 0.2) (layer F.Cu) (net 9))
 (segment (start 146.9 91.9) (end 147 91.8) (width 0.2) (layer F.Cu) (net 9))
 (segment (start 148.4 91.3) (end 147.8 91.3) (width 0.2) (layer F.Cu) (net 8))
 (segment (start 146.02805 90.55) (end 146.27805 90.3) (width 0.2) (layer F.Cu) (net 8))
 (segment (start 145 90.55) (end 146.02805 90.55) (width 0.2) (layer F.Cu) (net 8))
 (segment (start 146.27805 90.3) (end 148.4 90.3) (width 0.2) (layer F.Cu) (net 8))
 (segment (start 148.4 90.3) (end 148.6 90.5) (width 0.2) (layer F.Cu) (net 8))
 (segment (start 148.6 90.5) (end 148.6 91.1) (width 0.2) (layer F.Cu) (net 8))
 (segment (start 148.6 91.1) (end 148.4 91.3) (width 0.2) (layer F.Cu) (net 8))
 (segment (start 147.8 92.8) (end 149.65 92.8) (width 0.3) (layer F.Cu) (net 5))
 (segment (start 149.65 92.8) (end 150.2 92.25) (width 0.3) (layer F.Cu) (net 5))
 (via (at 150.2 90.45) (size 0.4) (drill 0.254) (layers F.Cu B.Cu) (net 5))
 (segment (start 150.2 92.25) (end 150.2 90.45) (width 0.3) (layer F.Cu) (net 5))
 (segment (start 158.155 86.995) (end 159.25 86.995) (width 0.3) (layer B.Cu) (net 5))
 (segment (start 150.2 90.45) (end 154.7 90.45) (width 0.3) (layer B.Cu) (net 5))
 (segment (start 154.7 90.45) (end 158.155 86.995) (width 0.3) (layer B.Cu) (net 5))
 (segment (start 152.4 91.8) (end 157.55 91.8) (width 0.3) (layer F.Cu) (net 3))
 (segment (start 157.825 92.075) (end 159.25 92.075) (width 0.3) (layer F.Cu) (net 3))
 (segment (start 157.55 91.8) (end 157.825 92.075) (width 0.3) (layer F.Cu) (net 3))
 (via (at 154.9 91.25) (size 0.4) (drill 0.254) (layers F.Cu B.Cu) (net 2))
 (segment (start 152.4 91.3) (end 154.85 91.3) (width 0.3) (layer F.Cu) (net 2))
 (segment (start 154.85 91.3) (end 154.9 91.25) (width 0.3) (layer F.Cu) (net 2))
 (segment (start 157.565 94.615) (end 159.25 94.615) (width 0.3) (layer B.Cu) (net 2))
 (segment (start 154.9 91.25) (end 154.9 91.95) (width 0.3) (layer B.Cu) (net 2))
 (segment (start 154.9 91.95) (end 157.565 94.615) (width 0.3) (layer B.Cu) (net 2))
 (via (at 149.45 92.05) (size 0.4) (drill 0.254) (layers F.Cu B.Cu) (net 6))
 (segment (start 147.8 92.3) (end 149.2 92.3) (width 0.3) (layer F.Cu) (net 6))
 (segment (start 149.2 92.3) (end 149.45 92.05) (width 0.3) (layer F.Cu) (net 6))
 (segment (start 158.205 97.155) (end 159.25 97.155) (width 0.3) (layer B.Cu) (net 6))
 (segment (start 155.5 94.45) (end 158.205 97.155) (width 0.3) (layer B.Cu) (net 6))
 (segment (start 149.45 92.05) (end 151.85 94.45) (width 0.3) (layer B.Cu) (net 6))
 (segment (start 151.85 94.45) (end 155.5 94.45) (width 0.3) (layer B.Cu) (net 6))
 (segment (start 152.95 85.9) (end 152.95 84.4) (width 0.4) (layer F.Cu) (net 11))
 (segment (start 143.9 83.75) (end 145.4 83.75) (width 0.6) (layer F.Cu) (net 16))
 (segment (start 153.05 95.6) (end 153.05 97.2) (width 0.3) (layer F.Cu) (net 10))
 (segment (start 152.4 92.8) (end 153.3 92.8) (width 0.3) (layer F.Cu) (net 4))
 (segment (start 154.75 94.25) (end 154.75 95.6) (width 0.3) (layer F.Cu) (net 4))
 (segment (start 153.3 92.8) (end 154.75 94.25) (width 0.3) (layer F.Cu) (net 4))
 (segment (start 152.4 92.3) (end 151.101 92.3) (width 0.3) (layer F.Cu) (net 1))
 (segment (start 151.101 92.3) (end 150.864 92.063) (width 0.3) (layer F.Cu) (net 1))
 (segment (start 152.4 90.8) (end 150.881 90.8) (width 0.3) (layer F.Cu) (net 1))
 (segment (start 150.881 90.8) (end 150.864 90.817) (width 0.3) (layer F.Cu) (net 1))
 (segment (start 150.864 92.063) (end 150.864 90.817) (width 0.3) (layer F.Cu) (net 1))
 (segment (start 150.864 90.817) (end 150.864 89.027) (width 0.3) (layer F.Cu) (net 1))
 (segment (start 150.864 89.027) (end 150.864 88.436) (width 0.6) (layer F.Cu) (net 1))
 (segment (start 151.05 88.25) (end 151.05 87.45) (width 0.6) (layer F.Cu) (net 1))
 (segment (start 150.864 88.436) (end 151.05 88.25) (width 0.6) (layer F.Cu) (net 1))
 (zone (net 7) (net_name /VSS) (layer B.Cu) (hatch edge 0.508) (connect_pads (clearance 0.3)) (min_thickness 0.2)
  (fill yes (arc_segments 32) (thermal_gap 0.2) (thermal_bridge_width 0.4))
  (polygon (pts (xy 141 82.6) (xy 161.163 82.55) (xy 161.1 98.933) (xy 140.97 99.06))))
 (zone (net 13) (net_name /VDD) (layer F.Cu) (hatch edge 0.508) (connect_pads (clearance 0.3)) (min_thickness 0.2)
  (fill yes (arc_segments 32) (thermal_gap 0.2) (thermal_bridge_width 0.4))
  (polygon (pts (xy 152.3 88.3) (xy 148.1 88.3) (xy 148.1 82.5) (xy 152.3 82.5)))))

